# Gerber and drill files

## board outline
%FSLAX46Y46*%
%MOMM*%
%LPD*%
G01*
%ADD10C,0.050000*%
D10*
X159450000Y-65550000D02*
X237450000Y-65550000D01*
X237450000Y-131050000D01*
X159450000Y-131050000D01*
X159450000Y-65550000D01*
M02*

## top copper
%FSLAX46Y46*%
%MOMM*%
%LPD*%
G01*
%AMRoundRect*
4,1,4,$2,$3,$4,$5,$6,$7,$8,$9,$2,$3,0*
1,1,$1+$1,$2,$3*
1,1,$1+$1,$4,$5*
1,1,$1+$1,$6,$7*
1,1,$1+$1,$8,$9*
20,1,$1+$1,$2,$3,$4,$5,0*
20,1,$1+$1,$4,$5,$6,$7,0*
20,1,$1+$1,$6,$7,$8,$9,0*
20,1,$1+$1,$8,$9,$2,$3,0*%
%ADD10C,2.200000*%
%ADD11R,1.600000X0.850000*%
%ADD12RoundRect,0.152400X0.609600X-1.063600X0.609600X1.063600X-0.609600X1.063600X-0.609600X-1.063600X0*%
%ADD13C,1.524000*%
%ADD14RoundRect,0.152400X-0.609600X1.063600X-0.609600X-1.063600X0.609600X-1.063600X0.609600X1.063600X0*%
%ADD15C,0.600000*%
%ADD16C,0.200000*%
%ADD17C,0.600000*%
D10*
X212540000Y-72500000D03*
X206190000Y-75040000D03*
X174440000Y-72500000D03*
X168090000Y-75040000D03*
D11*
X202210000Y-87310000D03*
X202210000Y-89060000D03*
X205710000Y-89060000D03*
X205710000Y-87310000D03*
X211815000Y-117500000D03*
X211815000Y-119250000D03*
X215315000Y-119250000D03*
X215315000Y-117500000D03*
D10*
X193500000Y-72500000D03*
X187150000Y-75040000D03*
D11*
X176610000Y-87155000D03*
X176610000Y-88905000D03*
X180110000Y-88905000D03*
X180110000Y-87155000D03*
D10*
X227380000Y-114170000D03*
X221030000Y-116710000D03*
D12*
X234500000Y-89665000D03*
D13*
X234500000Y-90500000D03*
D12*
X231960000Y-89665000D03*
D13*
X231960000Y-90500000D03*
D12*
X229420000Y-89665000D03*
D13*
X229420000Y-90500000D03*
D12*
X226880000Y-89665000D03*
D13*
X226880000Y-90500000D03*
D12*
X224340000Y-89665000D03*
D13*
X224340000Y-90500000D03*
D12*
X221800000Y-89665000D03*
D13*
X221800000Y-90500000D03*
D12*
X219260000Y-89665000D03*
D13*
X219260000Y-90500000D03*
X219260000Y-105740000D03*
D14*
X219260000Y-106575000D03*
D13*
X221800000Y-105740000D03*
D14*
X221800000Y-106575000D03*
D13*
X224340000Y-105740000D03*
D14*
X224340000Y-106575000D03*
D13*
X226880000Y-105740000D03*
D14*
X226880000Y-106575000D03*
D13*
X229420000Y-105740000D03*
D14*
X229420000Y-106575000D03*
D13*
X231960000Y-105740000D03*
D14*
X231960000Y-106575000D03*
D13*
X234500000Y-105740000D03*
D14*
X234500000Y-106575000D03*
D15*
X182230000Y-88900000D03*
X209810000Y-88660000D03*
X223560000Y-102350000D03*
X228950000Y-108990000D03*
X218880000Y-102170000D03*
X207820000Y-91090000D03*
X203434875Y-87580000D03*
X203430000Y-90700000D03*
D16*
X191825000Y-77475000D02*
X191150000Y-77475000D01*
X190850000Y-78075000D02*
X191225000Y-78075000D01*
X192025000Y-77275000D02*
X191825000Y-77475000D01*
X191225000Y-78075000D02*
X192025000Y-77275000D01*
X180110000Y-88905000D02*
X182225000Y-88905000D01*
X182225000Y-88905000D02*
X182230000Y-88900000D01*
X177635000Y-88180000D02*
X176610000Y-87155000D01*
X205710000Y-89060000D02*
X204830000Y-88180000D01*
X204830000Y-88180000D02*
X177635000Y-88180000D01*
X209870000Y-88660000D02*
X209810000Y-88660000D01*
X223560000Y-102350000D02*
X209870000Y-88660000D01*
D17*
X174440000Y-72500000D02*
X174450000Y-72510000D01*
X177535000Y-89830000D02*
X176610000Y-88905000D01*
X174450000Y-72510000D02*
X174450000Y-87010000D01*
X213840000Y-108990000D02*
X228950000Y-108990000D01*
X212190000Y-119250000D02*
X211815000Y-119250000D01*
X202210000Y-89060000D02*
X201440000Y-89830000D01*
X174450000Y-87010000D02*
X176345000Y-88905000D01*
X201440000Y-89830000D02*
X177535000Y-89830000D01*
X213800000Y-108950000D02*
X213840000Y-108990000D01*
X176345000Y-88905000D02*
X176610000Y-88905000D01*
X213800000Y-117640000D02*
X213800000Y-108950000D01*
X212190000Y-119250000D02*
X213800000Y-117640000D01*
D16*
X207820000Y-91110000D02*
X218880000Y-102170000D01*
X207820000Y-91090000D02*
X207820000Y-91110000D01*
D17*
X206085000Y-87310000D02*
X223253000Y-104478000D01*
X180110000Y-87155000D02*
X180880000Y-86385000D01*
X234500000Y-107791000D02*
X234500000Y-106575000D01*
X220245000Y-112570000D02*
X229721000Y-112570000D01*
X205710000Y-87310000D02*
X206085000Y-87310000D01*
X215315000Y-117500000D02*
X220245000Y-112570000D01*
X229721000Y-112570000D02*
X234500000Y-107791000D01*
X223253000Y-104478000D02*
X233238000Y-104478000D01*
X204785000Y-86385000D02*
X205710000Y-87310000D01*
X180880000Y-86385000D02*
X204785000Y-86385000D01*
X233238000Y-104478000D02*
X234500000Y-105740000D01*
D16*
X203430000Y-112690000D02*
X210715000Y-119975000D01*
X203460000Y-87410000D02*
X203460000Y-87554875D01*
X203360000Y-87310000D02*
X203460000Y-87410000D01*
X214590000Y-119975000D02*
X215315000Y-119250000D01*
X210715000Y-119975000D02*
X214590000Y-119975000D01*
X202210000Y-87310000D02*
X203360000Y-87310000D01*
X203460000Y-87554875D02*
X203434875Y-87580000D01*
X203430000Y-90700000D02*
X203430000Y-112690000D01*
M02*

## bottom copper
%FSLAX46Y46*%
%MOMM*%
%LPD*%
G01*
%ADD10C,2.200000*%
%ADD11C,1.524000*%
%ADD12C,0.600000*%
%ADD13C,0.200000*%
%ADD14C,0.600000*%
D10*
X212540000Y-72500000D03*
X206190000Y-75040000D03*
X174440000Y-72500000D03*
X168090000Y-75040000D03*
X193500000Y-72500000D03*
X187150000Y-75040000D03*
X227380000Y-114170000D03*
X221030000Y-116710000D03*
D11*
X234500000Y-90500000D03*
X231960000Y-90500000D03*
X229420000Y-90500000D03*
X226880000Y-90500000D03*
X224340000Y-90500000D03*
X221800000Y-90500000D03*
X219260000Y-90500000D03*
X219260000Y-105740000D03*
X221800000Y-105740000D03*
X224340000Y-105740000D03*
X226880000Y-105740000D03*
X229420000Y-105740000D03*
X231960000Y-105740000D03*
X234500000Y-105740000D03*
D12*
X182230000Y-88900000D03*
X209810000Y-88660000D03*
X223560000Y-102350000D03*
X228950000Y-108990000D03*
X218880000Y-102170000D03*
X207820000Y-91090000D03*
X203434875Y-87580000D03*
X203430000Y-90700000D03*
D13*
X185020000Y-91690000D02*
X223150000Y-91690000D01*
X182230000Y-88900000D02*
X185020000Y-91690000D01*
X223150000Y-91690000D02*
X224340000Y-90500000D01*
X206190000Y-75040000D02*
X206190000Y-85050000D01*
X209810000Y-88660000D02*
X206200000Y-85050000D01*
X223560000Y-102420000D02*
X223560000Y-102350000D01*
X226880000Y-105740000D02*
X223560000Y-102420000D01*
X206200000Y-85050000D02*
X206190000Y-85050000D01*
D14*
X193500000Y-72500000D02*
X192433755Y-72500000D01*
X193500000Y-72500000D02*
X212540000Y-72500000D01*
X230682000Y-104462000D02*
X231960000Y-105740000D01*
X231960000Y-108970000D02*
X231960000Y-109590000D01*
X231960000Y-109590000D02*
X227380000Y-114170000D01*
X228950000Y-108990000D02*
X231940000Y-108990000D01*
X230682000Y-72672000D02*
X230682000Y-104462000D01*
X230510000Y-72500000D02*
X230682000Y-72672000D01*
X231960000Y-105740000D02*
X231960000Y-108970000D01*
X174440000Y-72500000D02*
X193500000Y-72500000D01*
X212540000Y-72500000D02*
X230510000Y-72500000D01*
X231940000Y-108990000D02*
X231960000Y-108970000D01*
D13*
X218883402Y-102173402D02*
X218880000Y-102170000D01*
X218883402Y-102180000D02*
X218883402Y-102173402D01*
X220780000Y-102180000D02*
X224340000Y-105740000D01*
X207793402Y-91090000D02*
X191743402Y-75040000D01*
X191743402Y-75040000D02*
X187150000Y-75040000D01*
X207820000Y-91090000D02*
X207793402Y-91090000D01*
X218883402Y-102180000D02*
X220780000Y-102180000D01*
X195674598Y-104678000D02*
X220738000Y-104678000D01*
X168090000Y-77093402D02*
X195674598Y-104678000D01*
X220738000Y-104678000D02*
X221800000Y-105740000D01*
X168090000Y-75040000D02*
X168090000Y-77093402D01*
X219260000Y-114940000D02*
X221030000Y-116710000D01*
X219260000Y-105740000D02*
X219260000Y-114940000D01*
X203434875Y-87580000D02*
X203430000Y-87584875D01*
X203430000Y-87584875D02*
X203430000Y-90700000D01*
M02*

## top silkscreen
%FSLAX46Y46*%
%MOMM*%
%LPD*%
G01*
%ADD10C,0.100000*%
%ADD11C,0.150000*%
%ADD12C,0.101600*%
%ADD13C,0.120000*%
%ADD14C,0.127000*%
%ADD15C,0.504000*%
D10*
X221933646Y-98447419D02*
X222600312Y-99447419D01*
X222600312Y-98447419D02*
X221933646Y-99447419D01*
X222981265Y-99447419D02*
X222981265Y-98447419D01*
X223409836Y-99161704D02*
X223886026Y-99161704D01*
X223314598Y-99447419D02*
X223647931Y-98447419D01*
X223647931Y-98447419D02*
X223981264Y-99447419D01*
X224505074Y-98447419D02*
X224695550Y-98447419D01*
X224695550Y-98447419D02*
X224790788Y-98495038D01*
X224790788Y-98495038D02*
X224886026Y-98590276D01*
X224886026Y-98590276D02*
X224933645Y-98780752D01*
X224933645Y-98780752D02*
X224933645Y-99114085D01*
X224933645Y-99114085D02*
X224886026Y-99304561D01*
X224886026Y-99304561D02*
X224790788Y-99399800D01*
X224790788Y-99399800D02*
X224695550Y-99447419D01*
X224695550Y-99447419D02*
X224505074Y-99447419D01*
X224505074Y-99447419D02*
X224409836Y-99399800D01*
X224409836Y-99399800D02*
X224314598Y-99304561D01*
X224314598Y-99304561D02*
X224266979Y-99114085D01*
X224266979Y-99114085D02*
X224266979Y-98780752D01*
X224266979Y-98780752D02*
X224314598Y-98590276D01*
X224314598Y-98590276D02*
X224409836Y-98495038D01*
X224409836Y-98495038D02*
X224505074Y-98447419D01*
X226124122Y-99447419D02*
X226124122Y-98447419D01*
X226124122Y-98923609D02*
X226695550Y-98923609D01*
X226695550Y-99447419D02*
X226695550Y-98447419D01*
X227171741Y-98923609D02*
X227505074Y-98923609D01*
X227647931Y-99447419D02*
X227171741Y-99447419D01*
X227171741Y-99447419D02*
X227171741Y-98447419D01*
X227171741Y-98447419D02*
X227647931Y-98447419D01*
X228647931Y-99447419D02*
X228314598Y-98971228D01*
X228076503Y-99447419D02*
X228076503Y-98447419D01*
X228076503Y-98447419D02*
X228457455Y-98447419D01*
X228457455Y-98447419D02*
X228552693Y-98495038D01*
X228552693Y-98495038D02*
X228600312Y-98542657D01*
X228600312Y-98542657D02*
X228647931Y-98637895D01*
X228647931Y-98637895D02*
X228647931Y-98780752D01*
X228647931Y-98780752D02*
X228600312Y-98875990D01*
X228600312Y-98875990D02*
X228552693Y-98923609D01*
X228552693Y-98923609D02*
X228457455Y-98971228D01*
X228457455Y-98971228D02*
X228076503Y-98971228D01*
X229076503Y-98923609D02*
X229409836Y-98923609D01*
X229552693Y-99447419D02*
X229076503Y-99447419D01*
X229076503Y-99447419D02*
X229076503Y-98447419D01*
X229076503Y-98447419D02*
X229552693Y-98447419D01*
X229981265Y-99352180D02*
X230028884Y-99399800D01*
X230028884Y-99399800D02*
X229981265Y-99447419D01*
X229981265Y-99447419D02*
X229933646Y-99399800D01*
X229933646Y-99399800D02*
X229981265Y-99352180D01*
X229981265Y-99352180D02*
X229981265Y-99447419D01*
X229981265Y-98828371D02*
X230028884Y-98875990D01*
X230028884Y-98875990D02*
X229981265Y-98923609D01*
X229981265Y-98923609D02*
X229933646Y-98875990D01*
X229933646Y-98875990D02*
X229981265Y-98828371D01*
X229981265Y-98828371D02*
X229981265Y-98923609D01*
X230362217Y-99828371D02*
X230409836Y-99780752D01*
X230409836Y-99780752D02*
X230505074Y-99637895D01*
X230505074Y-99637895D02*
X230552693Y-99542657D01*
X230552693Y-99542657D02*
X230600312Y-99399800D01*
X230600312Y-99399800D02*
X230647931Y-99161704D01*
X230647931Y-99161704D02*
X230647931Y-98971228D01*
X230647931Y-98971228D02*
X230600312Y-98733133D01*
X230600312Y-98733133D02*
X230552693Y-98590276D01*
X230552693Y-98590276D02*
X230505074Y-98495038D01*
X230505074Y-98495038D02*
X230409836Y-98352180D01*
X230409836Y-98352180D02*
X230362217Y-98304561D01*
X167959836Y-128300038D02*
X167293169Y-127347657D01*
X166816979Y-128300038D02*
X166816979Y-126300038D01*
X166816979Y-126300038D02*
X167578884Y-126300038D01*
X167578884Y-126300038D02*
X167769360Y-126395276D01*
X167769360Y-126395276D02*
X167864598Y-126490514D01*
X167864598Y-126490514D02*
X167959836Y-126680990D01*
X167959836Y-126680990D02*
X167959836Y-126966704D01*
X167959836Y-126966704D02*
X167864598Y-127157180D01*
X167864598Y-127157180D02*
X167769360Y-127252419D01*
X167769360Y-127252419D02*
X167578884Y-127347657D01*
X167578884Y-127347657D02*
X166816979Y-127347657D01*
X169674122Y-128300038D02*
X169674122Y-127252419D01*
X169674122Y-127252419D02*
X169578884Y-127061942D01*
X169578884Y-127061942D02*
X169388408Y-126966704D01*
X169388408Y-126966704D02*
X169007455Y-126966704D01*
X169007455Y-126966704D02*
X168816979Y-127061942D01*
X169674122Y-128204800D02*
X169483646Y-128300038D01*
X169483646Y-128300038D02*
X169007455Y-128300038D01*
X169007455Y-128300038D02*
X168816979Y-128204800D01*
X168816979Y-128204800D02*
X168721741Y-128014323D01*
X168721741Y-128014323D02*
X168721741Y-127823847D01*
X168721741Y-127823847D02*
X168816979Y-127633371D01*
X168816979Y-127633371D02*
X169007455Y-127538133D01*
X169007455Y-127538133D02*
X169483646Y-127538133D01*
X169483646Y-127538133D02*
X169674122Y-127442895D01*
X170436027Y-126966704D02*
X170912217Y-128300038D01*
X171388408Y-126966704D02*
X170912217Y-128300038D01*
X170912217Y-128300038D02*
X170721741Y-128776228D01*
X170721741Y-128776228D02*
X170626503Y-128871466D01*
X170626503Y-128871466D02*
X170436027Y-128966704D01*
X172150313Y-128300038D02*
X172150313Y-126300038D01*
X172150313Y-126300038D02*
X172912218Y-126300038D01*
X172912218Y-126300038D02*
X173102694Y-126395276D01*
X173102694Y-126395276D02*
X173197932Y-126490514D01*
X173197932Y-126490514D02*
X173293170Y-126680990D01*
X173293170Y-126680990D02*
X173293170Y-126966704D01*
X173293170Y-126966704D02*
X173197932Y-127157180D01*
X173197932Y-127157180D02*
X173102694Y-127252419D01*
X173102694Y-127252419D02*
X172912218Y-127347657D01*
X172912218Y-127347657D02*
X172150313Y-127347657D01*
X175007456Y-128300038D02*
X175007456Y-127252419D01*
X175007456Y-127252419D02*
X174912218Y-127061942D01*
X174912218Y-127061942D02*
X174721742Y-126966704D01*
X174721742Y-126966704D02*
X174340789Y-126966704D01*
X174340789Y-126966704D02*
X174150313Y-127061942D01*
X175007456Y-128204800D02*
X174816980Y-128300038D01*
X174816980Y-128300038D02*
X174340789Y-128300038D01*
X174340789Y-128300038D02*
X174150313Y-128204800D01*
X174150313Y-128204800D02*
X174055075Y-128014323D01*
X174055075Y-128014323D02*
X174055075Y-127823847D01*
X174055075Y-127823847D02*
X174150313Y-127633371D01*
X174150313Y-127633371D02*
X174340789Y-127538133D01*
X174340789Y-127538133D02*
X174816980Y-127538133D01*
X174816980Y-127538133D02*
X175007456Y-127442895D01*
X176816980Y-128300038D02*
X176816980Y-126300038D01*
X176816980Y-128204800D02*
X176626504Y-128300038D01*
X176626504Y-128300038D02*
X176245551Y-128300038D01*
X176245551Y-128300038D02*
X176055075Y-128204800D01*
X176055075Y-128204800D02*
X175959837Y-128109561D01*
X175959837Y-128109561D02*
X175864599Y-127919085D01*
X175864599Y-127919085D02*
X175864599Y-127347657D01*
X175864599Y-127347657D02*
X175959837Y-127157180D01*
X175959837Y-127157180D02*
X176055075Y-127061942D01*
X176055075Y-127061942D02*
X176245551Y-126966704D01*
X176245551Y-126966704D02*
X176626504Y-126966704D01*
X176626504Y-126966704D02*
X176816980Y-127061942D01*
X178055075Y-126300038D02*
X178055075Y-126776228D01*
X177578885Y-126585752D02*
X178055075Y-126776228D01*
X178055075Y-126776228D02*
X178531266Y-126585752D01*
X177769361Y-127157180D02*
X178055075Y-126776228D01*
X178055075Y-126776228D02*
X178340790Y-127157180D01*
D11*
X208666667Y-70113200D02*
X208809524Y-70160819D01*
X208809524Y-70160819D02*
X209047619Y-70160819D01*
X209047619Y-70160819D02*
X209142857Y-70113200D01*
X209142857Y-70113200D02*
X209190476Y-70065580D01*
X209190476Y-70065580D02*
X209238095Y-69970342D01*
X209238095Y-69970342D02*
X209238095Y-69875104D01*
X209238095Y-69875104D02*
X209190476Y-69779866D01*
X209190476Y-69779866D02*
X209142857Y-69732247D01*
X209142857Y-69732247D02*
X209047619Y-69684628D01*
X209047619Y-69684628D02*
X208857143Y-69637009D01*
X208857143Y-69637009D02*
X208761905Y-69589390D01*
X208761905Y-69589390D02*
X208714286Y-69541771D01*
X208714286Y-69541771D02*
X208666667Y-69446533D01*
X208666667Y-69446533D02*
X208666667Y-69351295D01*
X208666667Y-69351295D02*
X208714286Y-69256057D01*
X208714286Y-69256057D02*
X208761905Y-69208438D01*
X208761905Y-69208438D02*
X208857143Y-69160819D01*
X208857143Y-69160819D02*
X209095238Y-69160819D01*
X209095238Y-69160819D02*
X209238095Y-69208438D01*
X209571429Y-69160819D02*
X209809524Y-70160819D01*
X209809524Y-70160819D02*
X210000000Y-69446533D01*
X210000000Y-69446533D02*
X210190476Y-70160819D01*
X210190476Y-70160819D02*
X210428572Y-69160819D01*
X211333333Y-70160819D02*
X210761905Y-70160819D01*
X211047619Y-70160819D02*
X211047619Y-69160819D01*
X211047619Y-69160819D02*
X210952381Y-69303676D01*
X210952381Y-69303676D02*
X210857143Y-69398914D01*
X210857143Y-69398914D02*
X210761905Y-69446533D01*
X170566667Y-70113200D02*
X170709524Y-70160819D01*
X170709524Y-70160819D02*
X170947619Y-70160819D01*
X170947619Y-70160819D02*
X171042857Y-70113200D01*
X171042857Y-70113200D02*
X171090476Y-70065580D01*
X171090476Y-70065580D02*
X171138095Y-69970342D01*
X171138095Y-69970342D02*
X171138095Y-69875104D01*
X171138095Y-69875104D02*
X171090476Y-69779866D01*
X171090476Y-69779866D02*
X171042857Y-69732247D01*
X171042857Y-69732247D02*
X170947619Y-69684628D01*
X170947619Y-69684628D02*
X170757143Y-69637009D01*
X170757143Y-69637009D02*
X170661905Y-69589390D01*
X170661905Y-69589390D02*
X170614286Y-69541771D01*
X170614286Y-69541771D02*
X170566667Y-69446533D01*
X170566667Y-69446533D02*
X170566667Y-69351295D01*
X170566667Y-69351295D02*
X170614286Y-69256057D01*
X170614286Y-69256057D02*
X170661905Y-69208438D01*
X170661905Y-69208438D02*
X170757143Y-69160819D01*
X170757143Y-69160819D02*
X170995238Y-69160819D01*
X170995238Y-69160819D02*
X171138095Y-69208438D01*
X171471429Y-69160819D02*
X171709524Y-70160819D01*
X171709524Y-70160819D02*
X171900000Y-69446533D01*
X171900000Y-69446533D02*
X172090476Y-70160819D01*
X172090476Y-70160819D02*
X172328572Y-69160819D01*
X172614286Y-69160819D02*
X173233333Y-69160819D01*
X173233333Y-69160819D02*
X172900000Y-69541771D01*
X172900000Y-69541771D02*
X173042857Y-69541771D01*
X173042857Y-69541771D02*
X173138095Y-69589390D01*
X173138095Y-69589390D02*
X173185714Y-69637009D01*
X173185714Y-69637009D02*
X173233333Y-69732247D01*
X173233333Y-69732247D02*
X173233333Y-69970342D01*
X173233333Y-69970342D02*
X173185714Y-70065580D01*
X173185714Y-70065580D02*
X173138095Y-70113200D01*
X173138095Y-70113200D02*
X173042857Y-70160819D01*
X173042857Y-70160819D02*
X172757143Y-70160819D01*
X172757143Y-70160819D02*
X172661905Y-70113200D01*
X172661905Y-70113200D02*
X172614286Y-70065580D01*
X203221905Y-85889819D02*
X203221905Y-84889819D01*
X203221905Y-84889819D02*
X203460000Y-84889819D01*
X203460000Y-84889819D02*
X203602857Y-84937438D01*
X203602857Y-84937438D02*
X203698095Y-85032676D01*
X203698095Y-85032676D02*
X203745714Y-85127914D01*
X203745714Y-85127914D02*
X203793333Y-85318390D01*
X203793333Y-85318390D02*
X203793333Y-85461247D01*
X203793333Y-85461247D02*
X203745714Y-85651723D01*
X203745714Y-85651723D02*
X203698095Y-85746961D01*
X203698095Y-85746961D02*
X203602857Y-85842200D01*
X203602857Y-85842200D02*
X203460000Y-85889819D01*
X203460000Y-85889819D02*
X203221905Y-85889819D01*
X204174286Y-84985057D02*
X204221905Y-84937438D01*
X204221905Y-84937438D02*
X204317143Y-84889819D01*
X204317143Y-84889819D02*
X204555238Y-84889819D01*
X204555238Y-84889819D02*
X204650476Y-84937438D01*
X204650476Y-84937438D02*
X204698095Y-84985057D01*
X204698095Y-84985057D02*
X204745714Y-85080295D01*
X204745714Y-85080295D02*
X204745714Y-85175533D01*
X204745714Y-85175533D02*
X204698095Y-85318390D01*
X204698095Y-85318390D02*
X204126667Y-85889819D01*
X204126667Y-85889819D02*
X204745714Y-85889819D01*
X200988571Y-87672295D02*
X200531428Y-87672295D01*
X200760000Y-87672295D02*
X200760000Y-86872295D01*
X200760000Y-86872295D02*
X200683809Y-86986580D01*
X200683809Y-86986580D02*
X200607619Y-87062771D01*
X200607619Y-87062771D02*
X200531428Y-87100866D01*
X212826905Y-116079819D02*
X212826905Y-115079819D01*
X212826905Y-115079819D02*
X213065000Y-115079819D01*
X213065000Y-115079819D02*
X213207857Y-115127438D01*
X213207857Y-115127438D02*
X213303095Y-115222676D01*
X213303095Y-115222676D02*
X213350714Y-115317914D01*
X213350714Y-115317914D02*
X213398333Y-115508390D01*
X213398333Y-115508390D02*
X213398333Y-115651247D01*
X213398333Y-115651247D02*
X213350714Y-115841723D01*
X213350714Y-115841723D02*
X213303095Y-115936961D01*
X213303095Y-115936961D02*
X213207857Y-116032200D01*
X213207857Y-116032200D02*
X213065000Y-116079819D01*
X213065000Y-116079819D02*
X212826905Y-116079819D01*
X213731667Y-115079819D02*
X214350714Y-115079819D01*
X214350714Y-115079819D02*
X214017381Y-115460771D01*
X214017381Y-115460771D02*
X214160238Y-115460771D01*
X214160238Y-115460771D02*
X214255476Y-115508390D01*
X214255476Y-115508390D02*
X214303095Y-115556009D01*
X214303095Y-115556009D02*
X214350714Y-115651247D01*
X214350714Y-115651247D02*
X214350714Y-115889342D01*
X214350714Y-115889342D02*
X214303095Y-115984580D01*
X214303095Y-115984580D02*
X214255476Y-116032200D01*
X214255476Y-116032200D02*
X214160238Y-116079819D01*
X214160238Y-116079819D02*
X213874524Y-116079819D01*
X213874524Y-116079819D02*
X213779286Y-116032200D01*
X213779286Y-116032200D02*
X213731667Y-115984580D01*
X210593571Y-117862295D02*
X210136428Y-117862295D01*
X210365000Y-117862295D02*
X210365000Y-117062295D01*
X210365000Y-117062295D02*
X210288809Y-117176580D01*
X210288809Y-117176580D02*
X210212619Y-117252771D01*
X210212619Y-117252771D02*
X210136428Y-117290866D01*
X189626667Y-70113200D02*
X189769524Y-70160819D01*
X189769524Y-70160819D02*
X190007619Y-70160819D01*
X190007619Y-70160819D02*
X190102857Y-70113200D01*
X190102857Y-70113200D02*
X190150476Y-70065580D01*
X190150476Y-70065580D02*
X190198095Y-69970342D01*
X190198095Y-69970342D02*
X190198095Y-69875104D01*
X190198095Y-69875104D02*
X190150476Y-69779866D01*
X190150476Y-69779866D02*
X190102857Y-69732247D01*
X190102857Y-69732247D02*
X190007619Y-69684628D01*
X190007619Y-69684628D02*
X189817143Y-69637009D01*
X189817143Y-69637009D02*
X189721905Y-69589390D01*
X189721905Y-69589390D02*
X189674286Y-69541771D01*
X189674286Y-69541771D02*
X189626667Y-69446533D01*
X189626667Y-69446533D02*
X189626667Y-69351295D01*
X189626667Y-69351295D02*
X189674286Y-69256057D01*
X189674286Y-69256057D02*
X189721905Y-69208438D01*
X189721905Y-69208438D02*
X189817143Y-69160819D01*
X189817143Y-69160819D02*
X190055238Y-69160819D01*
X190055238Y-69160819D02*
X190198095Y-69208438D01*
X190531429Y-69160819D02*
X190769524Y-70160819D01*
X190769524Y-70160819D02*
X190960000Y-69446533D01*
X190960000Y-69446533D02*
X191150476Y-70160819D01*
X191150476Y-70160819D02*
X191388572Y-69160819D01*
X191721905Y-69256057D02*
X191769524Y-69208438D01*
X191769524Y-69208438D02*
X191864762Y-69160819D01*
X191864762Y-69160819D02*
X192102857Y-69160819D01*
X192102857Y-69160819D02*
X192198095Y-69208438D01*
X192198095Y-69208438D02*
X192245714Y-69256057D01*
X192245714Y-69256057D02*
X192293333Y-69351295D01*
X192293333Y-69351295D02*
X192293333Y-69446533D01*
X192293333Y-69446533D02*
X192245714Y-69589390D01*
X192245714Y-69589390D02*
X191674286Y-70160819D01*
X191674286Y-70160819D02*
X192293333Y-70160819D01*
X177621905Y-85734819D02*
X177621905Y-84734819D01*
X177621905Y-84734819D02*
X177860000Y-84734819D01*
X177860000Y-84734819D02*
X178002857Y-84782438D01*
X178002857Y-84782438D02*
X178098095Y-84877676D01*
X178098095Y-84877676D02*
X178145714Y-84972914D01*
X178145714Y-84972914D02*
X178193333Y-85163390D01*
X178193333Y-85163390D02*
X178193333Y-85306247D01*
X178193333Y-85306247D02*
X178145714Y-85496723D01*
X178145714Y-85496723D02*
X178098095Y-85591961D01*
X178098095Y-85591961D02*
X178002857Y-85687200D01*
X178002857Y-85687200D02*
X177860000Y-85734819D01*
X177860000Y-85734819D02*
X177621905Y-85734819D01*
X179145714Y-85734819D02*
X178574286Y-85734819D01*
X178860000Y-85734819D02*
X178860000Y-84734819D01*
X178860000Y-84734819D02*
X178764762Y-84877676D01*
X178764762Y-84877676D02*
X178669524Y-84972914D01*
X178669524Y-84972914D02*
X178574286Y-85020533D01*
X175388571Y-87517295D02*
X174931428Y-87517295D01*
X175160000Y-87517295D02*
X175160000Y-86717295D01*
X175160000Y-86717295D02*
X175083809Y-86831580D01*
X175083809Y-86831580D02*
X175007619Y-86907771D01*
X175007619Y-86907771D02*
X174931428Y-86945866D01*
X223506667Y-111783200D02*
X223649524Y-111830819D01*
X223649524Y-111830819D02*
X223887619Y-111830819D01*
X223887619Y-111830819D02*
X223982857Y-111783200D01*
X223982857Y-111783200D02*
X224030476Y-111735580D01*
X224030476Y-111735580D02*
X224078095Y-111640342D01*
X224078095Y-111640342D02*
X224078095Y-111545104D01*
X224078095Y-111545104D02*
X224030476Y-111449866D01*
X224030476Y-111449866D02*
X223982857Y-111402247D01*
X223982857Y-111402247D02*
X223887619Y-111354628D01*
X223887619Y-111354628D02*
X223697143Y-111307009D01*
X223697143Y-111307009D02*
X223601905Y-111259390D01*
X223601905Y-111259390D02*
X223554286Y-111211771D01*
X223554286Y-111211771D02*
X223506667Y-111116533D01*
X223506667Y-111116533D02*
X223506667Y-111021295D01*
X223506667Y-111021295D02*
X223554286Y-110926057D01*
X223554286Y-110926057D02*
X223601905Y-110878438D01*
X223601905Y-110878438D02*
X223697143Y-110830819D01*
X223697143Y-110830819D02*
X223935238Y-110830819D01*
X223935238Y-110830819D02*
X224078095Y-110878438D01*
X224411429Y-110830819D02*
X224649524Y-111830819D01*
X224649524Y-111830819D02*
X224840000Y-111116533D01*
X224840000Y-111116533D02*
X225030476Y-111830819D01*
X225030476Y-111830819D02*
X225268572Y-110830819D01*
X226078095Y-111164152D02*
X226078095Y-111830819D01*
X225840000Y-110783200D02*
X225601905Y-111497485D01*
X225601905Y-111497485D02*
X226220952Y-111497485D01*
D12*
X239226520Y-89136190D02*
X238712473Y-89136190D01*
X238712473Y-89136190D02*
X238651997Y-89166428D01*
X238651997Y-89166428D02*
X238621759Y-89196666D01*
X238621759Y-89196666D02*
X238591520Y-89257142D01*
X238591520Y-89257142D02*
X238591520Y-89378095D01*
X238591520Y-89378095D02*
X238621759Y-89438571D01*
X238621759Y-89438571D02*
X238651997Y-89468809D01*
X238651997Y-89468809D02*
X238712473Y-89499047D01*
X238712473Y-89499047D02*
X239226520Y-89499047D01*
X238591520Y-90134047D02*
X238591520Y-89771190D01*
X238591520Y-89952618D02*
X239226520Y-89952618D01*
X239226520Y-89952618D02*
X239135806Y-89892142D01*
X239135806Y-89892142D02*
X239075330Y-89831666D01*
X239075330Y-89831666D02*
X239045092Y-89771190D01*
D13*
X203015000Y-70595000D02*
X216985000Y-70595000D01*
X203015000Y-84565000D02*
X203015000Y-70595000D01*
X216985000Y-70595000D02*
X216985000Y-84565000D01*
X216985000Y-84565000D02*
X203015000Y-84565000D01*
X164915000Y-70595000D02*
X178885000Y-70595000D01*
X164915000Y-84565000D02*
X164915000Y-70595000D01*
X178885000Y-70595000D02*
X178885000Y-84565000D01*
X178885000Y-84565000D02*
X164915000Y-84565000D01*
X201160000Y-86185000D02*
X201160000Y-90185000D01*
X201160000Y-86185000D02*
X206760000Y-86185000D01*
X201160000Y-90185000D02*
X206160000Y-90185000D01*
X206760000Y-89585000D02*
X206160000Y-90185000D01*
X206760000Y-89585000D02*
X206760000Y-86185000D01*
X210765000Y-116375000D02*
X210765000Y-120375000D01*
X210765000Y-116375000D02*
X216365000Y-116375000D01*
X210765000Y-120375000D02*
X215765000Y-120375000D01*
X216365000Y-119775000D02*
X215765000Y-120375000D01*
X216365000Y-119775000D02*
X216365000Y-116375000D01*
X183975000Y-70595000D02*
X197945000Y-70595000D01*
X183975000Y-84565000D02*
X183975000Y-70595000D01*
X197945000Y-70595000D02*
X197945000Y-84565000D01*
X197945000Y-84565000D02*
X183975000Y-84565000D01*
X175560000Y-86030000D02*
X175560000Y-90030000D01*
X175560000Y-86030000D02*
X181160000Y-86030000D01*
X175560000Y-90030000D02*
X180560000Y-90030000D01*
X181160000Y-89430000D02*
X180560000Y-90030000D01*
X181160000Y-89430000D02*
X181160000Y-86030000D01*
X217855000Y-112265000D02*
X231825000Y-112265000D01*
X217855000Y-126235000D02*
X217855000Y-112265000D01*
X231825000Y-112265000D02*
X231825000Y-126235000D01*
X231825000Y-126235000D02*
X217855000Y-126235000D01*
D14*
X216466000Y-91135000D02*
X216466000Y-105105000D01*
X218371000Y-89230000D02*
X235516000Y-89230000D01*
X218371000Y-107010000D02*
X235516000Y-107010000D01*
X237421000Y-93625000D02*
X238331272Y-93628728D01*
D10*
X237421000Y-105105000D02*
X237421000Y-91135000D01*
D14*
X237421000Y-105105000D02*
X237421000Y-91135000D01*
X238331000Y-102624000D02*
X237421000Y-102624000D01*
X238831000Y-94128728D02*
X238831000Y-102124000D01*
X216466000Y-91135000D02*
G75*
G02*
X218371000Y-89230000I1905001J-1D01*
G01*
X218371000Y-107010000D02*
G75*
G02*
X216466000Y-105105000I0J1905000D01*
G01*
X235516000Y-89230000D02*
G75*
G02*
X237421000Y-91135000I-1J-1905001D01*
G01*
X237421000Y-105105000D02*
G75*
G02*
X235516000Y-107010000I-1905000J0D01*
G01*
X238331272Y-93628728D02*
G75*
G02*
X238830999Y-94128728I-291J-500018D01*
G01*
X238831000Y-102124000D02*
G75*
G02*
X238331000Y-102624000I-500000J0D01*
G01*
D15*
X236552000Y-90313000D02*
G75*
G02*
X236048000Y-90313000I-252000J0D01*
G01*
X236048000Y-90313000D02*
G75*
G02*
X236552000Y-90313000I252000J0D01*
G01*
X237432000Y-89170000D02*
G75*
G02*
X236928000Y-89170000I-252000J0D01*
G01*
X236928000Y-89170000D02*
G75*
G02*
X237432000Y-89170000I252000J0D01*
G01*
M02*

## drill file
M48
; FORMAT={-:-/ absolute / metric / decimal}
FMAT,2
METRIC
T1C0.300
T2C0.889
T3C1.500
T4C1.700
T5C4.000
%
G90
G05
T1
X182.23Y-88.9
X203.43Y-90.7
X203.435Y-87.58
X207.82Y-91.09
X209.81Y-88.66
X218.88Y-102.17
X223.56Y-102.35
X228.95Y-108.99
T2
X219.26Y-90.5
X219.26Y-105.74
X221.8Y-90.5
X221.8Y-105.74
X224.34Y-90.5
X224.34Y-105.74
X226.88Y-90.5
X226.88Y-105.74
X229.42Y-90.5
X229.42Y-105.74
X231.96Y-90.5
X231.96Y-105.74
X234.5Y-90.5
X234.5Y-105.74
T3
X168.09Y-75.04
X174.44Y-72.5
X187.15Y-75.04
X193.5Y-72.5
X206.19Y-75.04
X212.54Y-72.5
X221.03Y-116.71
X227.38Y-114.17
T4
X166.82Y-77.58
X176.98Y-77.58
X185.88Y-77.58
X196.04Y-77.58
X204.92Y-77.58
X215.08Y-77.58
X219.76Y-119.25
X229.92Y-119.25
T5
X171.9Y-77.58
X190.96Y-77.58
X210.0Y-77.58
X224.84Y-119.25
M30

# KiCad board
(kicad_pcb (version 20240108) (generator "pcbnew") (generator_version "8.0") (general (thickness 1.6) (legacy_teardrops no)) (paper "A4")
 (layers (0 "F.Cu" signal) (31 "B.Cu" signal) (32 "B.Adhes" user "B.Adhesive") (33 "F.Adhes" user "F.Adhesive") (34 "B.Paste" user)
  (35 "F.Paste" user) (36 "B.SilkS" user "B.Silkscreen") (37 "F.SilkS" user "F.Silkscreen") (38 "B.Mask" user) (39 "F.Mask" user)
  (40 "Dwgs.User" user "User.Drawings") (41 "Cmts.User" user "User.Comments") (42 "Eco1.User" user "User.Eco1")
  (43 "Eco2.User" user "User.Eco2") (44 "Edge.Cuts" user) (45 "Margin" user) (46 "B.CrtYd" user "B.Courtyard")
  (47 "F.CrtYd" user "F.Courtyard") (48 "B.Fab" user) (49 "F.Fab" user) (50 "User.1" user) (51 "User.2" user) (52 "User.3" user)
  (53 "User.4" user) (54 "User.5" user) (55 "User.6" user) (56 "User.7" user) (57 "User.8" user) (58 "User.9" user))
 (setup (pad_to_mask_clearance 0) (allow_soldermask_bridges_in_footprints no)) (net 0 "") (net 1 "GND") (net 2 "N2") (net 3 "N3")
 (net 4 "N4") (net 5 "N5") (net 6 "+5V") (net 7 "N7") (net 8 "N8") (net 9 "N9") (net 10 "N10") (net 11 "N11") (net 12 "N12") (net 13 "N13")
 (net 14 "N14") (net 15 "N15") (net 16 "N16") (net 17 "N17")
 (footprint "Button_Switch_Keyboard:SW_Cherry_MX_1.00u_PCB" (layer "F.Cu") (at 212.54 72.5)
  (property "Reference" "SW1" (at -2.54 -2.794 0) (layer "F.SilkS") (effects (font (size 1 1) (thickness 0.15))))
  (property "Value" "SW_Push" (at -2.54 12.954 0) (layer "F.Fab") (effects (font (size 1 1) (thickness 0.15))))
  (fp_line (start -9.525 -1.905) (end 4.445 -1.905) (stroke (width 0.12) (type solid)) (layer "F.SilkS"))
  (fp_line (start -9.525 12.065) (end -9.525 -1.905) (stroke (width 0.12) (type solid)) (layer "F.SilkS"))
  (fp_line (start 4.445 -1.905) (end 4.445 12.065) (stroke (width 0.12) (type solid)) (layer "F.SilkS"))
  (fp_line (start 4.445 12.065) (end -9.525 12.065) (stroke (width 0.12) (type solid)) (layer "F.SilkS"))
  (pad "" np_thru_hole circle (at -7.62 5.08) (size 1.7 1.7) (drill 1.7) (layers "*.Cu" "*.Mask"))
  (pad "" np_thru_hole circle (at -2.54 5.08) (size 4 4) (drill 4) (layers "*.Cu" "*.Mask"))
  (pad "" np_thru_hole circle (at 2.54 5.08) (size 1.7 1.7) (drill 1.7) (layers "*.Cu" "*.Mask"))
  (pad "1" thru_hole circle (at 0 0) (size 2.2 2.2) (drill 1.5) (layers "*.Cu" "*.Mask") (remove_unused_layers no) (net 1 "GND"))
  (pad "2" thru_hole circle (at -6.35 2.54) (size 2.2 2.2) (drill 1.5) (layers "*.Cu" "*.Mask") (remove_unused_layers no) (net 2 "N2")))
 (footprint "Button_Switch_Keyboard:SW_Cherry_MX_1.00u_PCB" (layer "F.Cu") (at 174.44 72.5)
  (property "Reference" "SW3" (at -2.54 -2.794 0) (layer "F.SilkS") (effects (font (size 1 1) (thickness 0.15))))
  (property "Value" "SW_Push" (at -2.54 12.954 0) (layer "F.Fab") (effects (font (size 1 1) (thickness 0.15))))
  (fp_line (start -9.525 -1.905) (end 4.445 -1.905) (stroke (width 0.12) (type solid)) (layer "F.SilkS"))
  (fp_line (start -9.525 12.065) (end -9.525 -1.905) (stroke (width 0.12) (type solid)) (layer "F.SilkS"))
  (fp_line (start 4.445 -1.905) (end 4.445 12.065) (stroke (width 0.12) (type solid)) (layer "F.SilkS"))
  (fp_line (start 4.445 12.065) (end -9.525 12.065) (stroke (width 0.12) (type solid)) (layer "F.SilkS"))
  (pad "" np_thru_hole circle (at -7.62 5.08) (size 1.7 1.7) (drill 1.7) (layers "*.Cu" "*.Mask"))
  (pad "" np_thru_hole circle (at -2.54 5.08) (size 4 4) (drill 4) (layers "*.Cu" "*.Mask"))
  (pad "" np_thru_hole circle (at 2.54 5.08) (size 1.7 1.7) (drill 1.7) (layers "*.Cu" "*.Mask"))
  (pad "1" thru_hole circle (at 0 0) (size 2.2 2.2) (drill 1.5) (layers "*.Cu" "*.Mask") (remove_unused_layers no) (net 1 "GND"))
  (pad "2" thru_hole circle (at -6.35 2.54) (size 2.2 2.2) (drill 1.5) (layers "*.Cu" "*.Mask") (remove_unused_layers no) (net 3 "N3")))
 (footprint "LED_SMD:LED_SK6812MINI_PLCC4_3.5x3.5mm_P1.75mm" (layer "F.Cu") (at 203.96 88.185)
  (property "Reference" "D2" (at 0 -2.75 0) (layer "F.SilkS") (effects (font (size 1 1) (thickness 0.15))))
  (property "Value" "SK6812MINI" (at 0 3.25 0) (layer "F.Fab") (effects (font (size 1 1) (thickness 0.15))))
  (fp_line (start -2.8 -2) (end -2.8 2) (stroke (width 0.12) (type default)) (layer "F.SilkS"))
  (fp_line (start -2.8 -2) (end 2.8 -2) (stroke (width 0.12) (type solid)) (layer "F.SilkS"))
  (fp_line (start -2.8 2) (end 2.2 2) (stroke (width 0.12) (type solid)) (layer "F.SilkS"))
  (fp_line (start 2.8 1.4) (end 2.2 2) (stroke (width 0.12) (type default)) (layer "F.SilkS"))
  (fp_line (start 2.8 1.4) (end 2.8 -2) (stroke (width 0.12) (type solid)) (layer "F.SilkS"))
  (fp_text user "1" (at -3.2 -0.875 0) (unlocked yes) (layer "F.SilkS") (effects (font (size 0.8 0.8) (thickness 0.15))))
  (pad "1" smd rect (at -1.75 -0.875) (size 1.6 0.85) (layers "F.Cu" "F.Paste" "F.Mask") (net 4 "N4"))
  (pad "2" smd rect (at -1.75 0.875) (size 1.6 0.85) (layers "F.Cu" "F.Paste" "F.Mask") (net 1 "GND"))
  (pad "3" smd rect (at 1.75 0.875) (size 1.6 0.85) (layers "F.Cu" "F.Paste" "F.Mask") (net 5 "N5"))
  (pad "4" smd rect (at 1.75 -0.875) (size 1.6 0.85) (layers "F.Cu" "F.Paste" "F.Mask") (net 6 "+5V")))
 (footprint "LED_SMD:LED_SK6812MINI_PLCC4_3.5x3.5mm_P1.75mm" (layer "F.Cu") (at 213.565 118.375)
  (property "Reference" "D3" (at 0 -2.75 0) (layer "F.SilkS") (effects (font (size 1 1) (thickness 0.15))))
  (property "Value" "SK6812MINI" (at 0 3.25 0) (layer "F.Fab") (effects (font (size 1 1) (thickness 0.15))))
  (fp_line (start -2.8 -2) (end -2.8 2) (stroke (width 0.12) (type default)) (layer "F.SilkS"))
  (fp_line (start -2.8 -2) (end 2.8 -2) (stroke (width 0.12) (type solid)) (layer "F.SilkS"))
  (fp_line (start -2.8 2) (end 2.2 2) (stroke (width 0.12) (type solid)) (layer "F.SilkS"))
  (fp_line (start 2.8 1.4) (end 2.2 2) (stroke (width 0.12) (type default)) (layer "F.SilkS"))
  (fp_line (start 2.8 1.4) (end 2.8 -2) (stroke (width 0.12) (type solid)) (layer "F.SilkS"))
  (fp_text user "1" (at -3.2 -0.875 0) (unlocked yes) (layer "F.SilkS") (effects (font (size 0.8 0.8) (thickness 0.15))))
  (pad "1" smd rect (at -1.75 -0.875) (size 1.6 0.85) (layers "F.Cu" "F.Paste" "F.Mask") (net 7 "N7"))
  (pad "2" smd rect (at -1.75 0.875) (size 1.6 0.85) (layers "F.Cu" "F.Paste" "F.Mask") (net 1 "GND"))
  (pad "3" smd rect (at 1.75 0.875) (size 1.6 0.85) (layers "F.Cu" "F.Paste" "F.Mask") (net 4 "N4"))
  (pad "4" smd rect (at 1.75 -0.875) (size 1.6 0.85) (layers "F.Cu" "F.Paste" "F.Mask") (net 6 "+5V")))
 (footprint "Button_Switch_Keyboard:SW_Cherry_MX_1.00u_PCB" (layer "F.Cu") (at 193.5 72.5)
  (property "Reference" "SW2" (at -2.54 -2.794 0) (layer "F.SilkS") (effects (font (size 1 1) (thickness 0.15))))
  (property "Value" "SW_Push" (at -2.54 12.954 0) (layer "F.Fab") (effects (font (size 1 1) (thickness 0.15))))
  (fp_line (start -9.525 -1.905) (end 4.445 -1.905) (stroke (width 0.12) (type solid)) (layer "F.SilkS"))
  (fp_line (start -9.525 12.065) (end -9.525 -1.905) (stroke (width 0.12) (type solid)) (layer "F.SilkS"))
  (fp_line (start 4.445 -1.905) (end 4.445 12.065) (stroke (width 0.12) (type solid)) (layer "F.SilkS"))
  (fp_line (start 4.445 12.065) (end -9.525 12.065) (stroke (width 0.12) (type solid)) (layer "F.SilkS"))
  (pad "" np_thru_hole circle (at -7.62 5.08) (size 1.7 1.7) (drill 1.7) (layers "*.Cu" "*.Mask"))
  (pad "" np_thru_hole circle (at -2.54 5.08) (size 4 4) (drill 4) (layers "*.Cu" "*.Mask"))
  (pad "" np_thru_hole circle (at 2.54 5.08) (size 1.7 1.7) (drill 1.7) (layers "*.Cu" "*.Mask"))
  (pad "1" thru_hole circle (at 0 0) (size 2.2 2.2) (drill 1.5) (layers "*.Cu" "*.Mask") (remove_unused_layers no) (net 1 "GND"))
  (pad "2" thru_hole circle (at -6.35 2.54) (size 2.2 2.2) (drill 1.5) (layers "*.Cu" "*.Mask") (remove_unused_layers no) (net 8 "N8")))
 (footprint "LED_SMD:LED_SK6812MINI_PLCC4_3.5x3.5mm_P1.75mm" (layer "F.Cu") (at 178.36 88.03)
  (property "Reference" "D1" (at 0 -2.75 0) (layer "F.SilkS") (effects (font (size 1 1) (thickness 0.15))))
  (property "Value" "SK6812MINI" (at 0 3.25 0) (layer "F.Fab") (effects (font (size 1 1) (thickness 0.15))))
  (fp_line (start -2.8 -2) (end -2.8 2) (stroke (width 0.12) (type default)) (layer "F.SilkS"))
  (fp_line (start -2.8 -2) (end 2.8 -2) (stroke (width 0.12) (type solid)) (layer "F.SilkS"))
  (fp_line (start -2.8 2) (end 2.2 2) (stroke (width 0.12) (type solid)) (layer "F.SilkS"))
  (fp_line (start 2.8 1.4) (end 2.2 2) (stroke (width 0.12) (type default)) (layer "F.SilkS"))
  (fp_line (start 2.8 1.4) (end 2.8 -2) (stroke (width 0.12) (type solid)) (layer "F.SilkS"))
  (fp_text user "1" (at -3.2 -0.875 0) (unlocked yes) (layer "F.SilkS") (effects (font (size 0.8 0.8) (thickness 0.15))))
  (pad "1" smd rect (at -1.75 -0.875) (size 1.6 0.85) (layers "F.Cu" "F.Paste" "F.Mask") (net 5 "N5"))
  (pad "2" smd rect (at -1.75 0.875) (size 1.6 0.85) (layers "F.Cu" "F.Paste" "F.Mask") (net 1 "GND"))
  (pad "3" smd rect (at 1.75 0.875) (size 1.6 0.85) (layers "F.Cu" "F.Paste" "F.Mask") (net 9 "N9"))
  (pad "4" smd rect (at 1.75 -0.875) (size 1.6 0.85) (layers "F.Cu" "F.Paste" "F.Mask") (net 6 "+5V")))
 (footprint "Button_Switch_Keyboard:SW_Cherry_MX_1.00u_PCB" (layer "F.Cu") (at 227.38 114.17)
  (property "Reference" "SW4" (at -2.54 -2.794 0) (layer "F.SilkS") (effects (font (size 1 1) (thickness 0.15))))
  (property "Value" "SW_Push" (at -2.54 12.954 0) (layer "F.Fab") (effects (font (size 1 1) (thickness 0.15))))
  (fp_line (start -9.525 -1.905) (end 4.445 -1.905) (stroke (width 0.12) (type solid)) (layer "F.SilkS"))
  (fp_line (start -9.525 12.065) (end -9.525 -1.905) (stroke (width 0.12) (type solid)) (layer "F.SilkS"))
  (fp_line (start 4.445 -1.905) (end 4.445 12.065) (stroke (width 0.12) (type solid)) (layer "F.SilkS"))
  (fp_line (start 4.445 12.065) (end -9.525 12.065) (stroke (width 0.12) (type solid)) (layer "F.SilkS"))
  (pad "" np_thru_hole circle (at -7.62 5.08) (size 1.7 1.7) (drill 1.7) (layers "*.Cu" "*.Mask"))
  (pad "" np_thru_hole circle (at -2.54 5.08) (size 4 4) (drill 4) (layers "*.Cu" "*.Mask"))
  (pad "" np_thru_hole circle (at 2.54 5.08) (size 1.7 1.7) (drill 1.7) (layers "*.Cu" "*.Mask"))
  (pad "1" thru_hole circle (at 0 0) (size 2.2 2.2) (drill 1.5) (layers "*.Cu" "*.Mask") (remove_unused_layers no) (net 1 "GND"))
  (pad "2" thru_hole circle (at -6.35 2.54) (size 2.2 2.2) (drill 1.5) (layers "*.Cu" "*.Mask") (remove_unused_layers no) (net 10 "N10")))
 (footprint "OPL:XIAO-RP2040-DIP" (layer "F.Cu") (at 226.88 98.12 -90)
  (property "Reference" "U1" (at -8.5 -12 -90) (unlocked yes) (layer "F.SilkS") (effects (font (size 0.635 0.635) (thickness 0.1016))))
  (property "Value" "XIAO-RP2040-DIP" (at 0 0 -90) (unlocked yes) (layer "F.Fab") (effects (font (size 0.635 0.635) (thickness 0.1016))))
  (fp_line (start -6.985 10.414) (end 6.985 10.414) (stroke (width 0.127) (type solid)) (layer "F.SilkS"))
  (fp_line (start -8.89 8.509) (end -8.89 -8.636) (stroke (width 0.127) (type solid)) (layer "F.SilkS"))
  (fp_line (start 8.89 8.509) (end 8.89 -8.636) (stroke (width 0.127) (type solid)) (layer "F.SilkS"))
  (fp_line (start -4.495 -10.541) (end -4.491272 -11.451272) (stroke (width 0.127) (type solid)) (layer "F.SilkS"))
  (fp_line (start 6.985 -10.541) (end -6.985 -10.541) (stroke (width 0.1) (type solid)) (layer "F.SilkS"))
  (fp_line (start 6.985 -10.541) (end -6.985 -10.541) (stroke (width 0.127) (type solid)) (layer "F.SilkS"))
  (fp_line (start 4.504 -11.451) (end 4.504 -10.541) (stroke (width 0.127) (type solid)) (layer "F.SilkS"))
  (fp_line (start -3.991272 -11.951) (end 4.004 -11.951) (stroke (width 0.127) (type solid)) (layer "F.SilkS"))
  (fp_arc (start -6.985 10.414) (mid -8.332038 9.856038) (end -8.89 8.509) (stroke (width 0.127) (type solid)) (layer "F.SilkS"))
  (fp_arc (start 8.89 8.509) (mid 8.332038 9.856038) (end 6.985 10.414) (stroke (width 0.127) (type solid)) (layer "F.SilkS"))
  (fp_arc (start -8.89 -8.636) (mid -8.332038 -9.983038) (end -6.985 -10.541) (stroke (width 0.127) (type solid)) (layer "F.SilkS"))
  (fp_arc (start 6.985 -10.541) (mid 8.332038 -9.983038) (end 8.89 -8.636) (stroke (width 0.127) (type solid)) (layer "F.SilkS"))
  (fp_arc (start -4.491272 -11.451272) (mid -4.344724 -11.804644) (end -3.991272 -11.951) (stroke (width 0.127) (type default))
   (layer "F.SilkS"))
  (fp_arc (start 4.004 -11.951) (mid 4.357553 -11.804553) (end 4.504 -11.451) (stroke (width 0.127) (type default)) (layer "F.SilkS"))
  (fp_circle (center -7.807 -9.42) (end -7.807 -9.674) (stroke (width 0.5) (type solid)) (fill solid) (layer "F.SilkS"))
  (fp_circle (center -8.95 -10.3) (end -8.95 -10.554) (stroke (width 0.5) (type solid)) (fill solid) (layer "F.SilkS"))
  (pad "1" smd roundrect (at -8.455 -7.62 90) (size 2.432 1.524) (layers "F.Cu" "F.Mask") (roundrect_rratio 0.1) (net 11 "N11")
   (thermal_bridge_angle 45))
  (pad "1" thru_hole circle (at -7.62 -7.62 90) (size 1.524 1.524) (drill 0.889) (layers "*.Cu" "*.Mask") (remove_unused_layers no)
   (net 11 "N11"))
  (pad "2" smd roundrect (at -8.455 -5.08 90) (size 2.432 1.524) (layers "F.Cu" "F.Mask") (roundrect_rratio 0.1) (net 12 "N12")
   (thermal_bridge_angle 45))
  (pad "2" thru_hole circle (at -7.62 -5.08 90) (size 1.524 1.524) (drill 0.889) (layers "*.Cu" "*.Mask") (remove_unused_layers no)
   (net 12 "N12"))
  (pad "3" smd roundrect (at -8.455 -2.54 90) (size 2.432 1.524) (layers "F.Cu" "F.Mask") (roundrect_rratio 0.1) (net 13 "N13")
   (thermal_bridge_angle 45))
  (pad "3" thru_hole circle (at -7.62 -2.54 90) (size 1.524 1.524) (drill 0.889) (layers "*.Cu" "*.Mask") (remove_unused_layers no)
   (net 13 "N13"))
  (pad "4" smd roundrect (at -8.455 0 90) (size 2.432 1.524) (layers "F.Cu" "F.Mask") (roundrect_rratio 0.1) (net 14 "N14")
   (thermal_bridge_angle 45))
  (pad "4" thru_hole circle (at -7.62 0 90) (size 1.524 1.524) (drill 0.889) (layers "*.Cu" "*.Mask") (remove_unused_layers no)
   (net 14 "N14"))
  (pad "5" smd roundrect (at -8.455 2.54 90) (size 2.432 1.524) (layers "F.Cu" "F.Mask") (roundrect_rratio 0.1) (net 9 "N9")
   (thermal_bridge_angle 45))
  (pad "5" thru_hole circle (at -7.62 2.54 90) (size 1.524 1.524) (drill 0.889) (layers "*.Cu" "*.Mask") (remove_unused_layers no)
   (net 9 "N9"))
  (pad "6" smd roundrect (at -8.455 5.08 90) (size 2.432 1.524) (layers "F.Cu" "F.Mask") (roundrect_rratio 0.1) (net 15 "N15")
   (thermal_bridge_angle 45))
  (pad "6" thru_hole circle (at -7.62 5.08 90) (size 1.524 1.524) (drill 0.889) (layers "*.Cu" "*.Mask") (remove_unused_layers no)
   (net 15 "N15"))
  (pad "7" smd roundrect (at -8.455 7.62 90) (size 2.432 1.524) (layers "F.Cu" "F.Mask") (roundrect_rratio 0.1) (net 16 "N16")
   (thermal_bridge_angle 45))
  (pad "7" thru_hole circle (at -7.62 7.62 90) (size 1.524 1.524) (drill 0.889) (layers "*.Cu" "*.Mask") (remove_unused_layers no)
   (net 16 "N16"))
  (pad "8" thru_hole circle (at 7.62 7.62 270) (size 1.524 1.524) (drill 0.889) (layers "*.Cu" "*.Mask") (remove_unused_layers no)
   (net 10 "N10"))
  (pad "8" smd roundrect (at 8.455 7.62 270) (size 2.432 1.524) (layers "F.Cu" "F.Mask") (roundrect_rratio 0.1) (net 10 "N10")
   (thermal_bridge_angle 45))
  (pad "9" thru_hole circle (at 7.62 5.08 270) (size 1.524 1.524) (drill 0.889) (layers "*.Cu" "*.Mask") (remove_unused_layers no)
   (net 3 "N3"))
  (pad "9" smd roundrect (at 8.455 5.08 270) (size 2.432 1.524) (layers "F.Cu" "F.Mask") (roundrect_rratio 0.1) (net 3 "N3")
   (thermal_bridge_angle 45))
  (pad "10" thru_hole circle (at 7.62 2.54 270) (size 1.524 1.524) (drill 0.889) (layers "*.Cu" "*.Mask") (remove_unused_layers no)
   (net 8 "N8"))
  (pad "10" smd roundrect (at 8.455 2.54 270) (size 2.432 1.524) (layers "F.Cu" "F.Mask") (roundrect_rratio 0.1) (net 8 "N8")
   (thermal_bridge_angle 45))
  (pad "11" thru_hole circle (at 7.62 0 270) (size 1.524 1.524) (drill 0.889) (layers "*.Cu" "*.Mask") (remove_unused_layers no)
   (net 2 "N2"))
  (pad "11" smd roundrect (at 8.455 0 270) (size 2.432 1.524) (layers "F.Cu" "F.Mask") (roundrect_rratio 0.1) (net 2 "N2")
   (thermal_bridge_angle 45))
  (pad "12" thru_hole circle (at 7.62 -2.54 270) (size 1.524 1.524) (drill 0.889) (layers "*.Cu" "*.Mask") (remove_unused_layers no)
   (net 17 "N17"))
  (pad "12" smd roundrect (at 8.455 -2.54 270) (size 2.432 1.524) (layers "F.Cu" "F.Mask") (roundrect_rratio 0.1) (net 17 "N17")
   (thermal_bridge_angle 45))
  (pad "13" thru_hole circle (at 7.62 -5.08 270) (size 1.524 1.524) (drill 0.889) (layers "*.Cu" "*.Mask") (remove_unused_layers no)
   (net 1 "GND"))
  (pad "13" smd roundrect (at 8.455 -5.08 270) (size 2.432 1.524) (layers "F.Cu" "F.Mask") (roundrect_rratio 0.1) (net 1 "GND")
   (thermal_bridge_angle 45))
  (pad "14" thru_hole circle (at 7.62 -7.62 270) (size 1.524 1.524) (drill 0.889) (layers "*.Cu" "*.Mask") (remove_unused_layers no)
   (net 6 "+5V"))
  (pad "14" smd roundrect (at 8.455 -7.62 270) (size 2.432 1.524) (layers "F.Cu" "F.Mask") (roundrect_rratio 0.1) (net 6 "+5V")
   (thermal_bridge_angle 45)))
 (gr_rect (start 159.45 65.55) (end 237.45 131.05) (stroke (width 0.05) (type default)) (fill none) (layer "Edge.Cuts"))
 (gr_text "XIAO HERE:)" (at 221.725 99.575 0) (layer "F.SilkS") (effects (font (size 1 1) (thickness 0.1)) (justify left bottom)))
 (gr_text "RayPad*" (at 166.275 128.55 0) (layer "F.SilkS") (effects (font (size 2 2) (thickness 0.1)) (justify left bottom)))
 (segment (start 191.825 77.475) (end 191.15 77.475) (width 0.2) (layer "F.Cu") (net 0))
 (segment (start 190.85 78.075) (end 191.225 78.075) (width 0.2) (layer "F.Cu") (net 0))
 (segment (start 192.025 77.275) (end 191.825 77.475) (width 0.2) (layer "F.Cu") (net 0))
 (segment (start 191.225 78.075) (end 192.025 77.275) (width 0.2) (layer "F.Cu") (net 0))
 (segment (start 180.11 88.905) (end 182.225 88.905) (width 0.2) (layer "F.Cu") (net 9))
 (segment (start 182.225 88.905) (end 182.23 88.9) (width 0.2) (layer "F.Cu") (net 9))
 (via (at 182.23 88.9) (size 0.6) (drill 0.3) (layers "F.Cu" "B.Cu") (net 9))
 (segment (start 185.02 91.69) (end 223.15 91.69) (width 0.2) (layer "B.Cu") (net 9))
 (segment (start 182.23 88.9) (end 185.02 91.69) (width 0.2) (layer "B.Cu") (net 9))
 (segment (start 223.15 91.69) (end 224.34 90.5) (width 0.2) (layer "B.Cu") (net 9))
 (segment (start 177.635 88.18) (end 176.61 87.155) (width 0.2) (layer "F.Cu") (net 5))
 (segment (start 205.71 89.06) (end 204.83 88.18) (width 0.2) (layer "F.Cu") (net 5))
 (segment (start 204.83 88.18) (end 177.635 88.18) (width 0.2) (layer "F.Cu") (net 5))
 (segment (start 209.87 88.66) (end 209.81 88.66) (width 0.2) (layer "F.Cu") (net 2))
 (segment (start 223.56 102.35) (end 209.87 88.66) (width 0.2) (layer "F.Cu") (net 2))
 (via (at 209.81 88.66) (size 0.6) (drill 0.3) (layers "F.Cu" "B.Cu") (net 2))
 (via (at 223.56 102.35) (size 0.6) (drill 0.3) (layers "F.Cu" "B.Cu") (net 2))
 (segment (start 206.19 75.04) (end 206.19 85.05) (width 0.2) (layer "B.Cu") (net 2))
 (segment (start 209.81 88.66) (end 206.2 85.05) (width 0.2) (layer "B.Cu") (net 2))
 (segment (start 223.56 102.42) (end 223.56 102.35) (width 0.2) (layer "B.Cu") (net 2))
 (segment (start 226.88 105.74) (end 223.56 102.42) (width 0.2) (layer "B.Cu") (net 2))
 (segment (start 206.2 85.05) (end 206.19 85.05) (width 0.2) (layer "B.Cu") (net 2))
 (segment (start 174.44 72.5) (end 174.45 72.51) (width 0.6) (layer "F.Cu") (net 1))
 (segment (start 177.535 89.83) (end 176.61 88.905) (width 0.6) (layer "F.Cu") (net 1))
 (segment (start 174.45 72.51) (end 174.45 87.01) (width 0.6) (layer "F.Cu") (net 1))
 (segment (start 213.84 108.99) (end 228.95 108.99) (width 0.6) (layer "F.Cu") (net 1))
 (segment (start 212.19 119.25) (end 211.815 119.25) (width 0.6) (layer "F.Cu") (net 1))
 (segment (start 202.21 89.06) (end 201.44 89.83) (width 0.6) (layer "F.Cu") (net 1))
 (segment (start 174.45 87.01) (end 176.345 88.905) (width 0.6) (layer "F.Cu") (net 1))
 (segment (start 201.44 89.83) (end 177.535 89.83) (width 0.6) (layer "F.Cu") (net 1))
 (segment (start 213.8 108.95) (end 213.84 108.99) (width 0.6) (layer "F.Cu") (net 1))
 (segment (start 176.345 88.905) (end 176.61 88.905) (width 0.6) (layer "F.Cu") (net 1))
 (segment (start 213.8 117.64) (end 213.8 108.95) (width 0.6) (layer "F.Cu") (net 1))
 (segment (start 212.19 119.25) (end 213.8 117.64) (width 0.6) (layer "F.Cu") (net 1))
 (via (at 228.95 108.99) (size 0.6) (drill 0.3) (layers "F.Cu" "B.Cu") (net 1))
 (segment (start 193.5 72.5) (end 192.433755 72.5) (width 0.6) (layer "B.Cu") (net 1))
 (segment (start 193.5 72.5) (end 212.54 72.5) (width 0.6) (layer "B.Cu") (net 1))
 (segment (start 230.682 104.462) (end 231.96 105.74) (width 0.6) (layer "B.Cu") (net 1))
 (segment (start 231.96 108.97) (end 231.96 109.59) (width 0.6) (layer "B.Cu") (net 1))
 (segment (start 231.96 109.59) (end 227.38 114.17) (width 0.6) (layer "B.Cu") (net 1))
 (segment (start 228.95 108.99) (end 231.94 108.99) (width 0.6) (layer "B.Cu") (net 1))
 (segment (start 230.682 72.672) (end 230.682 104.462) (width 0.6) (layer "B.Cu") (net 1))
 (segment (start 230.51 72.5) (end 230.682 72.672) (width 0.6) (layer "B.Cu") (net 1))
 (segment (start 231.96 105.74) (end 231.96 108.97) (width 0.6) (layer "B.Cu") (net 1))
 (segment (start 174.44 72.5) (end 193.5 72.5) (width 0.6) (layer "B.Cu") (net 1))
 (segment (start 212.54 72.5) (end 230.51 72.5) (width 0.6) (layer "B.Cu") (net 1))
 (segment (start 231.94 108.99) (end 231.96 108.97) (width 0.6) (layer "B.Cu") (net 1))
 (segment (start 207.82 91.11) (end 218.88 102.17) (width 0.2) (layer "F.Cu") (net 8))
 (segment (start 207.82 91.09) (end 207.82 91.11) (width 0.2) (layer "F.Cu") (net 8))
 (via (at 218.88 102.17) (size 0.6) (drill 0.3) (layers "F.Cu" "B.Cu") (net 8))
 (via (at 207.82 91.09) (size 0.6) (drill 0.3) (layers "F.Cu" "B.Cu") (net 8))
 (segment (start 218.883402 102.173402) (end 218.88 102.17) (width 0.2) (layer "B.Cu") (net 8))
 (segment (start 218.883402 102.18) (end 218.883402 102.173402) (width 0.2) (layer "B.Cu") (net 8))
 (segment (start 220.78 102.18) (end 224.34 105.74) (width 0.2) (layer "B.Cu") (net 8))
 (segment (start 207.793402 91.09) (end 191.743402 75.04) (width 0.2) (layer "B.Cu") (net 8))
 (segment (start 191.743402 75.04) (end 187.15 75.04) (width 0.2) (layer "B.Cu") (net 8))
 (segment (start 207.82 91.09) (end 207.793402 91.09) (width 0.2) (layer "B.Cu") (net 8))
 (segment (start 218.883402 102.18) (end 220.78 102.18) (width 0.2) (layer "B.Cu") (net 8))
 (segment (start 195.674598 104.678) (end 220.738 104.678) (width 0.2) (layer "B.Cu") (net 3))
 (segment (start 168.09 77.093402) (end 195.674598 104.678) (width 0.2) (layer "B.Cu") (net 3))
 (segment (start 220.738 104.678) (end 221.8 105.74) (width 0.2) (layer "B.Cu") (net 3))
 (segment (start 168.09 75.04) (end 168.09 77.093402) (width 0.2) (layer "B.Cu") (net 3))
 (segment (start 219.26 114.94) (end 221.03 116.71) (width 0.2) (layer "B.Cu") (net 10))
 (segment (start 219.26 105.74) (end 219.26 114.94) (width 0.2) (layer "B.Cu") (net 10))
 (segment (start 206.085 87.31) (end 223.253 104.478) (width 0.6) (layer "F.Cu") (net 6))
 (segment (start 180.11 87.155) (end 180.88 86.385) (width 0.6) (layer "F.Cu") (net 6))
 (segment (start 234.5 107.791) (end 234.5 106.575) (width 0.6) (layer "F.Cu") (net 6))
 (segment (start 220.245 112.57) (end 229.721 112.57) (width 0.6) (layer "F.Cu") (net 6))
 (segment (start 205.71 87.31) (end 206.085 87.31) (width 0.6) (layer "F.Cu") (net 6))
 (segment (start 215.315 117.5) (end 220.245 112.57) (width 0.6) (layer "F.Cu") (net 6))
 (segment (start 229.721 112.57) (end 234.5 107.791) (width 0.6) (layer "F.Cu") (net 6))
 (segment (start 223.253 104.478) (end 233.238 104.478) (width 0.6) (layer "F.Cu") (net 6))
 (segment (start 204.785 86.385) (end 205.71 87.31) (width 0.6) (layer "F.Cu") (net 6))
 (segment (start 180.88 86.385) (end 204.785 86.385) (width 0.6) (layer "F.Cu") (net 6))
 (segment (start 233.238 104.478) (end 234.5 105.74) (width 0.6) (layer "F.Cu") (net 6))
 (segment (start 203.43 112.69) (end 210.715 119.975) (width 0.2) (layer "F.Cu") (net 4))
 (segment (start 203.46 87.41) (end 203.46 87.554875) (width 0.2) (layer "F.Cu") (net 4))
 (segment (start 203.36 87.31) (end 203.46 87.41) (width 0.2) (layer "F.Cu") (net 4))
 (segment (start 214.59 119.975) (end 215.315 119.25) (width 0.2) (layer "F.Cu") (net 4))
 (segment (start 210.715 119.975) (end 214.59 119.975) (width 0.2) (layer "F.Cu") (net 4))
 (segment (start 202.21 87.31) (end 203.36 87.31) (width 0.2) (layer "F.Cu") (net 4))
 (segment (start 203.46 87.554875) (end 203.434875 87.58) (width 0.2) (layer "F.Cu") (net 4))
 (segment (start 203.43 90.7) (end 203.43 112.69) (width 0.2) (layer "F.Cu") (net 4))
 (via (at 203.434875 87.58) (size 0.6) (drill 0.3) (layers "F.Cu" "B.Cu") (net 4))
 (via (at 203.43 90.7) (size 0.6) (drill 0.3) (layers "F.Cu" "B.Cu") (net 4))
 (segment (start 203.434875 87.58) (end 203.43 87.584875) (width 0.2) (layer "B.Cu") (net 4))
 (segment (start 203.43 87.584875) (end 203.43 90.7) (width 0.2) (layer "B.Cu") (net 4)))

